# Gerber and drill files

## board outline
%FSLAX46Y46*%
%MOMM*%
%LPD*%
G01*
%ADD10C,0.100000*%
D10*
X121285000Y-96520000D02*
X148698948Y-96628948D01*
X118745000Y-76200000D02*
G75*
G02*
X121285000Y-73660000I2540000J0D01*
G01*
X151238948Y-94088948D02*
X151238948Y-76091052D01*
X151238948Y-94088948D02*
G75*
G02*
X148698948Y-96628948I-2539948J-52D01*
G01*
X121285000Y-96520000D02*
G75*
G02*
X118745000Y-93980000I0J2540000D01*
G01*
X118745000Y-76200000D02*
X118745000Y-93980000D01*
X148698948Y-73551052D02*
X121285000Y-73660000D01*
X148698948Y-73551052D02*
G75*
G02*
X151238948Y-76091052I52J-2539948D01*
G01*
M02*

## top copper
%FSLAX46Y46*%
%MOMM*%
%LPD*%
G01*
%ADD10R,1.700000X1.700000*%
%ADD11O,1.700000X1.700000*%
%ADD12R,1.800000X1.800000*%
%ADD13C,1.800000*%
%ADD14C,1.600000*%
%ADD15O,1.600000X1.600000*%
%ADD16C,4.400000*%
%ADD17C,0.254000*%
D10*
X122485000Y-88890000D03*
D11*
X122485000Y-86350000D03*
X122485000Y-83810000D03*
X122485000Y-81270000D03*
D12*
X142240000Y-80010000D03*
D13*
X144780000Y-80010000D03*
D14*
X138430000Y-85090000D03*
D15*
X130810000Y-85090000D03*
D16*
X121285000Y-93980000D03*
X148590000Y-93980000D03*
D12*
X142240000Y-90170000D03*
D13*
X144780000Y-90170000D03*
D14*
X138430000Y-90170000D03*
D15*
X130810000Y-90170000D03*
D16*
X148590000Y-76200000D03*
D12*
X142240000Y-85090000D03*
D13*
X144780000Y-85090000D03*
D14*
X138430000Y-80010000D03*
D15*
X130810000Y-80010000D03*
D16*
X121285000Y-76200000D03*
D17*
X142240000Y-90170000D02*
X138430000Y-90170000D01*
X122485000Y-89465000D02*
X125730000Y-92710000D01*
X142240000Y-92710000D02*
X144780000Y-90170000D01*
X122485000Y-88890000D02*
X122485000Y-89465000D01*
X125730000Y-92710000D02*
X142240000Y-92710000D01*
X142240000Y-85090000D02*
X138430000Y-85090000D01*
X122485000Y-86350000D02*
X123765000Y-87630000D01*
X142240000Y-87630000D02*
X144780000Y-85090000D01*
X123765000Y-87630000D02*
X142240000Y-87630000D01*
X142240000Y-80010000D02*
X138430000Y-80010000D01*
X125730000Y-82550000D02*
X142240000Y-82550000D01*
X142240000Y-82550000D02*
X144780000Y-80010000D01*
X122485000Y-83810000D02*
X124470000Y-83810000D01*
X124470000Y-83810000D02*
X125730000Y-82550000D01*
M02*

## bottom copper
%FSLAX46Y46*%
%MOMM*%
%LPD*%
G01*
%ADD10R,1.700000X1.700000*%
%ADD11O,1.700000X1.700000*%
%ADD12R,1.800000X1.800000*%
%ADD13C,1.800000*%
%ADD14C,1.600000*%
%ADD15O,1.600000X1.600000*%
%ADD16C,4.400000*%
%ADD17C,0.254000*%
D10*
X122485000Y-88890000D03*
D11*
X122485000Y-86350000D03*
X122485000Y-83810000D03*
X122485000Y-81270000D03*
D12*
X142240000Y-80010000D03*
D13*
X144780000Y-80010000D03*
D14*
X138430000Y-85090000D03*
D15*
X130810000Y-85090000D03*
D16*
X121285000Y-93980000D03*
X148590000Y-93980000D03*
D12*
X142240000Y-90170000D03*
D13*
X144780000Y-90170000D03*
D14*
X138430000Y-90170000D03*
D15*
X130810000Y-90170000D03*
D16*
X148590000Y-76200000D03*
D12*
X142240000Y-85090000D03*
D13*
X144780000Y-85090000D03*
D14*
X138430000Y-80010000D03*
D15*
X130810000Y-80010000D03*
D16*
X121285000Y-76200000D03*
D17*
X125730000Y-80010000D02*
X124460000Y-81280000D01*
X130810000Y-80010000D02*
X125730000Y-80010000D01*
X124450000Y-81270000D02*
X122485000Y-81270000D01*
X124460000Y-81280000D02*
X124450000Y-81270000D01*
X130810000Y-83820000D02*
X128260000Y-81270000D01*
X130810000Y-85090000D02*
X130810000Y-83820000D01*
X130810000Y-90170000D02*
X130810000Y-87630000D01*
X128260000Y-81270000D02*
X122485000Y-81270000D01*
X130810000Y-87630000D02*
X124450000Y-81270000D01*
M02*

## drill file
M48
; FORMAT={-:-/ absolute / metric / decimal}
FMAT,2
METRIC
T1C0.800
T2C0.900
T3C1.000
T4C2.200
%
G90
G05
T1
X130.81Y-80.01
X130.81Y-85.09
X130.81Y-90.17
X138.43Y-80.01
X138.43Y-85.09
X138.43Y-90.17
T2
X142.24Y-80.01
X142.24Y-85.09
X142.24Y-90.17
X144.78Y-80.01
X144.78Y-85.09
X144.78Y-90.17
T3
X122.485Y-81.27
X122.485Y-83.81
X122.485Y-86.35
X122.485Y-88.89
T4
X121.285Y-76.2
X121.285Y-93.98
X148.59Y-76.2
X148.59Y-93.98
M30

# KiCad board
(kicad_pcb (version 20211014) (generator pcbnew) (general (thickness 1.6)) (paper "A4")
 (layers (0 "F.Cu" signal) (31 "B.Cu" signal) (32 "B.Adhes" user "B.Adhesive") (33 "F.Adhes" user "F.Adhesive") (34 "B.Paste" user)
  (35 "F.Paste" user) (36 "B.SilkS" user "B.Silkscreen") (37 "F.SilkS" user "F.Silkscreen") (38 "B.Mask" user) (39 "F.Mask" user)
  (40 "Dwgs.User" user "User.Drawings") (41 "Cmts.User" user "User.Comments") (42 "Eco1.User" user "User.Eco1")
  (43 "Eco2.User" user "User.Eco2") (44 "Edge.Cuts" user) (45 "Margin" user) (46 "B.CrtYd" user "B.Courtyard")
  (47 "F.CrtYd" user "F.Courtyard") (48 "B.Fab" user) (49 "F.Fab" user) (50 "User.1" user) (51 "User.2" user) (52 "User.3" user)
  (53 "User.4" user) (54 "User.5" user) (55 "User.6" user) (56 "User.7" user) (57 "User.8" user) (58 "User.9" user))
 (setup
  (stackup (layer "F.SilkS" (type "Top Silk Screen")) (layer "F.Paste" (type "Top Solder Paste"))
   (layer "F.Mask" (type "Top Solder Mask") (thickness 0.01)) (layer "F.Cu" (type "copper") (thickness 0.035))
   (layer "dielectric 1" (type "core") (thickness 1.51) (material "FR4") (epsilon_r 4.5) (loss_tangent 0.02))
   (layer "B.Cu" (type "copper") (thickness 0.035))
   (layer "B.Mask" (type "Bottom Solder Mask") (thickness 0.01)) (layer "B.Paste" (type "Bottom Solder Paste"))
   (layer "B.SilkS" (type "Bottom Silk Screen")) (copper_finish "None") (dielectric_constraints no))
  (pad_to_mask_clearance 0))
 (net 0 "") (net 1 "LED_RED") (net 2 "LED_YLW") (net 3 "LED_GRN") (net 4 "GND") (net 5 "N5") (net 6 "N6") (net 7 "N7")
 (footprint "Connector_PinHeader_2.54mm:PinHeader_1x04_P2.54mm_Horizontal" (layer "F.Cu") (at 122.485 88.89 180)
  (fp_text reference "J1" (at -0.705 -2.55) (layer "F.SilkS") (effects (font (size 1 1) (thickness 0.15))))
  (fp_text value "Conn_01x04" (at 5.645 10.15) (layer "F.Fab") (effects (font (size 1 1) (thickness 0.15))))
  (pad "1" thru_hole rect (at 0 0 180) (size 1.7 1.7) (drill 1) (layers *.Cu *.Mask) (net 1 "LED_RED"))
  (pad "2" thru_hole oval (at 0 2.54 180) (size 1.7 1.7) (drill 1) (layers *.Cu *.Mask) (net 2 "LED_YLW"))
  (pad "3" thru_hole oval (at 0 5.08 180) (size 1.7 1.7) (drill 1) (layers *.Cu *.Mask) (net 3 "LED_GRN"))
  (pad "4" thru_hole oval (at 0 7.62 180) (size 1.7 1.7) (drill 1) (layers *.Cu *.Mask) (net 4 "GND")))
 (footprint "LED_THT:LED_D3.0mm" (layer "F.Cu") (at 142.24 80.01)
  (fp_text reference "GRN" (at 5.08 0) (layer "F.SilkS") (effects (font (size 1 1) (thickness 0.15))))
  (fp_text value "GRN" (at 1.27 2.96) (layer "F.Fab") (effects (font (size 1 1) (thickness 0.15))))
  (pad "1" thru_hole rect (at 0 0) (size 1.8 1.8) (drill 0.9) (layers *.Cu *.Mask) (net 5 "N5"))
  (pad "2" thru_hole circle (at 2.54 0) (size 1.8 1.8) (drill 0.9) (layers *.Cu *.Mask) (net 3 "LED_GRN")))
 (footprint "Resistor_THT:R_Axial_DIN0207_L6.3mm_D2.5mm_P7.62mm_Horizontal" (layer "F.Cu") (at 138.43 85.09 180)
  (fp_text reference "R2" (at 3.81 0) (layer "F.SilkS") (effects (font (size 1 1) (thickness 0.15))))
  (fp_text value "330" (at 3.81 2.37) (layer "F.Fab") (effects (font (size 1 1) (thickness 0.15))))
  (pad "1" thru_hole circle (at 0 0 180) (size 1.6 1.6) (drill 0.8) (layers *.Cu *.Mask) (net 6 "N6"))
  (pad "2" thru_hole oval (at 7.62 0 180) (size 1.6 1.6) (drill 0.8) (layers *.Cu *.Mask) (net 4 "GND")))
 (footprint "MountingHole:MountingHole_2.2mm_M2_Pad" (layer "F.Cu") (at 121.285 93.98)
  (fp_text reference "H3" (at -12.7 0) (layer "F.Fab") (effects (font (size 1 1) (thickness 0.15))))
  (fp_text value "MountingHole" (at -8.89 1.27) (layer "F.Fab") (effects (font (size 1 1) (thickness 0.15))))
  (pad "1" thru_hole circle (at 0 0) (size 4.4 4.4) (drill 2.2) (layers *.Cu *.Mask)))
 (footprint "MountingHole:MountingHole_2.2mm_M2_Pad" (layer "F.Cu") (at 148.59 93.98)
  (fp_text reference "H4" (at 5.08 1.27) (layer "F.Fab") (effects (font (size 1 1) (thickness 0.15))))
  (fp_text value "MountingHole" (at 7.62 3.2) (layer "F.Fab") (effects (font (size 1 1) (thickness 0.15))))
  (pad "1" thru_hole circle (at 0 0) (size 4.4 4.4) (drill 2.2) (layers *.Cu *.Mask)))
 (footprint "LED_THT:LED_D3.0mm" (layer "F.Cu") (at 142.24 90.17)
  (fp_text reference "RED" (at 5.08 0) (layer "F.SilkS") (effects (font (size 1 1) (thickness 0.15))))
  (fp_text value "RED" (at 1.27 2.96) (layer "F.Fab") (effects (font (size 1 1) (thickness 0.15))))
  (pad "1" thru_hole rect (at 0 0) (size 1.8 1.8) (drill 0.9) (layers *.Cu *.Mask) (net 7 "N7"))
  (pad "2" thru_hole circle (at 2.54 0) (size 1.8 1.8) (drill 0.9) (layers *.Cu *.Mask) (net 1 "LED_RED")))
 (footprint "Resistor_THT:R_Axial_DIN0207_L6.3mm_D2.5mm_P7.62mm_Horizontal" (layer "F.Cu") (at 138.43 90.17 180)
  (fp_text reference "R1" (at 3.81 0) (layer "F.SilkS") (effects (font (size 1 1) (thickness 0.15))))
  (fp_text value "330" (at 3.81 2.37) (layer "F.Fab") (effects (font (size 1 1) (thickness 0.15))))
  (pad "1" thru_hole circle (at 0 0 180) (size 1.6 1.6) (drill 0.8) (layers *.Cu *.Mask) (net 7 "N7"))
  (pad "2" thru_hole oval (at 7.62 0 180) (size 1.6 1.6) (drill 0.8) (layers *.Cu *.Mask) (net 4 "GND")))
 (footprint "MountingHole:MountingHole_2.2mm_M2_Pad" (layer "F.Cu") (at 148.59 76.2)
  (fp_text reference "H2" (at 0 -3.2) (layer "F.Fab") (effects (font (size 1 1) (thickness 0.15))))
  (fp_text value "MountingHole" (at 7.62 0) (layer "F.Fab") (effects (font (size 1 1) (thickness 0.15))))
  (pad "1" thru_hole circle (at 0 0) (size 4.4 4.4) (drill 2.2) (layers *.Cu *.Mask)))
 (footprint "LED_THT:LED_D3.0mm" (layer "F.Cu") (at 142.24 85.09)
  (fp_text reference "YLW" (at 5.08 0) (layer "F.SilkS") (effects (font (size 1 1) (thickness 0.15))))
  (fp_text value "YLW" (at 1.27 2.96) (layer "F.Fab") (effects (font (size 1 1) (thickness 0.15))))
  (pad "1" thru_hole rect (at 0 0) (size 1.8 1.8) (drill 0.9) (layers *.Cu *.Mask) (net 6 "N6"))
  (pad "2" thru_hole circle (at 2.54 0) (size 1.8 1.8) (drill 0.9) (layers *.Cu *.Mask) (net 2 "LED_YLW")))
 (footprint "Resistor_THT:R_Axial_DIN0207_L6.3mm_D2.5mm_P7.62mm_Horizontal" (layer "F.Cu") (at 138.43 80.01 180)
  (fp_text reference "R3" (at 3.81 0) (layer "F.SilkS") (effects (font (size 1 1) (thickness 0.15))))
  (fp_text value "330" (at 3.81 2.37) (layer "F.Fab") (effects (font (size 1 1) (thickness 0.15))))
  (pad "1" thru_hole circle (at 0 0 180) (size 1.6 1.6) (drill 0.8) (layers *.Cu *.Mask) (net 5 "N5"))
  (pad "2" thru_hole oval (at 7.62 0 180) (size 1.6 1.6) (drill 0.8) (layers *.Cu *.Mask) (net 4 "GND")))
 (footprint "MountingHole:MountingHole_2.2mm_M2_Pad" (layer "F.Cu") (at 121.285 76.2)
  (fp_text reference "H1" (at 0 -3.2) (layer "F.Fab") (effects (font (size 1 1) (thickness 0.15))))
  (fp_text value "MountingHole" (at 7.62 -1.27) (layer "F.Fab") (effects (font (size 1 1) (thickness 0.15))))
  (pad "1" thru_hole circle (at 0 0) (size 4.4 4.4) (drill 2.2) (layers *.Cu *.Mask)))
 (gr_line (start 121.285 96.52) (end 148.698948 96.628948) (layer "Edge.Cuts") (width 0.1))
 (gr_arc (start 118.745 76.2) (mid 119.488949 74.403949) (end 121.285 73.66) (layer "Edge.Cuts") (width 0.1))
 (gr_line (start 151.238948 94.088948) (end 151.238948 76.091052) (layer "Edge.Cuts") (width 0.1))
 (gr_arc (start 151.238948 94.088948) (mid 150.495 95.885) (end 148.698948 96.628948) (layer "Edge.Cuts") (width 0.1))
 (gr_arc (start 121.285 96.52) (mid 119.488949 95.776051) (end 118.745 93.98) (layer "Edge.Cuts") (width 0.1))
 (gr_line (start 118.745 76.2) (end 118.745 93.98) (layer "Edge.Cuts") (width 0.1))
 (gr_line (start 148.698948 73.551052) (end 121.285 73.66) (layer "Edge.Cuts") (width 0.1))
 (gr_arc (start 148.698948 73.551052) (mid 150.495 74.295) (end 151.238948 76.091052) (layer "Edge.Cuts") (width 0.1))
 (segment (start 142.24 90.17) (end 138.43 90.17) (width 0.254) (layer "F.Cu") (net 7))
 (segment (start 122.485 89.465) (end 125.73 92.71) (width 0.254) (layer "F.Cu") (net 1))
 (segment (start 142.24 92.71) (end 144.78 90.17) (width 0.254) (layer "F.Cu") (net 1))
 (segment (start 122.485 88.89) (end 122.485 89.465) (width 0.254) (layer "F.Cu") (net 1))
 (segment (start 125.73 92.71) (end 142.24 92.71) (width 0.254) (layer "F.Cu") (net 1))
 (segment (start 142.24 85.09) (end 138.43 85.09) (width 0.254) (layer "F.Cu") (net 6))
 (segment (start 122.485 86.35) (end 123.765 87.63) (width 0.254) (layer "F.Cu") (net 2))
 (segment (start 142.24 87.63) (end 144.78 85.09) (width 0.254) (layer "F.Cu") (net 2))
 (segment (start 123.765 87.63) (end 142.24 87.63) (width 0.254) (layer "F.Cu") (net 2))
 (segment (start 142.24 80.01) (end 138.43 80.01) (width 0.254) (layer "F.Cu") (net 5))
 (segment (start 125.73 82.55) (end 142.24 82.55) (width 0.254) (layer "F.Cu") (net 3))
 (segment (start 142.24 82.55) (end 144.78 80.01) (width 0.254) (layer "F.Cu") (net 3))
 (segment (start 122.485 83.81) (end 124.47 83.81) (width 0.254) (layer "F.Cu") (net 3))
 (segment (start 124.47 83.81) (end 125.73 82.55) (width 0.254) (layer "F.Cu") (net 3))
 (segment (start 125.73 80.01) (end 124.46 81.28) (width 0.254) (layer "B.Cu") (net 4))
 (segment (start 130.81 80.01) (end 125.73 80.01) (width 0.254) (layer "B.Cu") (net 4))
 (segment (start 124.45 81.27) (end 122.485 81.27) (width 0.254) (layer "B.Cu") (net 4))
 (segment (start 124.46 81.28) (end 124.45 81.27) (width 0.254) (layer "B.Cu") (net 4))
 (segment (start 130.81 83.82) (end 128.26 81.27) (width 0.254) (layer "B.Cu") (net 4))
 (segment (start 130.81 85.09) (end 130.81 83.82) (width 0.254) (layer "B.Cu") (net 4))
 (segment (start 130.81 90.17) (end 130.81 87.63) (width 0.254) (layer "B.Cu") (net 4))
 (segment (start 128.26 81.27) (end 122.485 81.27) (width 0.254) (layer "B.Cu") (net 4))
 (segment (start 130.81 87.63) (end 124.45 81.27) (width 0.254) (layer "B.Cu") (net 4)))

